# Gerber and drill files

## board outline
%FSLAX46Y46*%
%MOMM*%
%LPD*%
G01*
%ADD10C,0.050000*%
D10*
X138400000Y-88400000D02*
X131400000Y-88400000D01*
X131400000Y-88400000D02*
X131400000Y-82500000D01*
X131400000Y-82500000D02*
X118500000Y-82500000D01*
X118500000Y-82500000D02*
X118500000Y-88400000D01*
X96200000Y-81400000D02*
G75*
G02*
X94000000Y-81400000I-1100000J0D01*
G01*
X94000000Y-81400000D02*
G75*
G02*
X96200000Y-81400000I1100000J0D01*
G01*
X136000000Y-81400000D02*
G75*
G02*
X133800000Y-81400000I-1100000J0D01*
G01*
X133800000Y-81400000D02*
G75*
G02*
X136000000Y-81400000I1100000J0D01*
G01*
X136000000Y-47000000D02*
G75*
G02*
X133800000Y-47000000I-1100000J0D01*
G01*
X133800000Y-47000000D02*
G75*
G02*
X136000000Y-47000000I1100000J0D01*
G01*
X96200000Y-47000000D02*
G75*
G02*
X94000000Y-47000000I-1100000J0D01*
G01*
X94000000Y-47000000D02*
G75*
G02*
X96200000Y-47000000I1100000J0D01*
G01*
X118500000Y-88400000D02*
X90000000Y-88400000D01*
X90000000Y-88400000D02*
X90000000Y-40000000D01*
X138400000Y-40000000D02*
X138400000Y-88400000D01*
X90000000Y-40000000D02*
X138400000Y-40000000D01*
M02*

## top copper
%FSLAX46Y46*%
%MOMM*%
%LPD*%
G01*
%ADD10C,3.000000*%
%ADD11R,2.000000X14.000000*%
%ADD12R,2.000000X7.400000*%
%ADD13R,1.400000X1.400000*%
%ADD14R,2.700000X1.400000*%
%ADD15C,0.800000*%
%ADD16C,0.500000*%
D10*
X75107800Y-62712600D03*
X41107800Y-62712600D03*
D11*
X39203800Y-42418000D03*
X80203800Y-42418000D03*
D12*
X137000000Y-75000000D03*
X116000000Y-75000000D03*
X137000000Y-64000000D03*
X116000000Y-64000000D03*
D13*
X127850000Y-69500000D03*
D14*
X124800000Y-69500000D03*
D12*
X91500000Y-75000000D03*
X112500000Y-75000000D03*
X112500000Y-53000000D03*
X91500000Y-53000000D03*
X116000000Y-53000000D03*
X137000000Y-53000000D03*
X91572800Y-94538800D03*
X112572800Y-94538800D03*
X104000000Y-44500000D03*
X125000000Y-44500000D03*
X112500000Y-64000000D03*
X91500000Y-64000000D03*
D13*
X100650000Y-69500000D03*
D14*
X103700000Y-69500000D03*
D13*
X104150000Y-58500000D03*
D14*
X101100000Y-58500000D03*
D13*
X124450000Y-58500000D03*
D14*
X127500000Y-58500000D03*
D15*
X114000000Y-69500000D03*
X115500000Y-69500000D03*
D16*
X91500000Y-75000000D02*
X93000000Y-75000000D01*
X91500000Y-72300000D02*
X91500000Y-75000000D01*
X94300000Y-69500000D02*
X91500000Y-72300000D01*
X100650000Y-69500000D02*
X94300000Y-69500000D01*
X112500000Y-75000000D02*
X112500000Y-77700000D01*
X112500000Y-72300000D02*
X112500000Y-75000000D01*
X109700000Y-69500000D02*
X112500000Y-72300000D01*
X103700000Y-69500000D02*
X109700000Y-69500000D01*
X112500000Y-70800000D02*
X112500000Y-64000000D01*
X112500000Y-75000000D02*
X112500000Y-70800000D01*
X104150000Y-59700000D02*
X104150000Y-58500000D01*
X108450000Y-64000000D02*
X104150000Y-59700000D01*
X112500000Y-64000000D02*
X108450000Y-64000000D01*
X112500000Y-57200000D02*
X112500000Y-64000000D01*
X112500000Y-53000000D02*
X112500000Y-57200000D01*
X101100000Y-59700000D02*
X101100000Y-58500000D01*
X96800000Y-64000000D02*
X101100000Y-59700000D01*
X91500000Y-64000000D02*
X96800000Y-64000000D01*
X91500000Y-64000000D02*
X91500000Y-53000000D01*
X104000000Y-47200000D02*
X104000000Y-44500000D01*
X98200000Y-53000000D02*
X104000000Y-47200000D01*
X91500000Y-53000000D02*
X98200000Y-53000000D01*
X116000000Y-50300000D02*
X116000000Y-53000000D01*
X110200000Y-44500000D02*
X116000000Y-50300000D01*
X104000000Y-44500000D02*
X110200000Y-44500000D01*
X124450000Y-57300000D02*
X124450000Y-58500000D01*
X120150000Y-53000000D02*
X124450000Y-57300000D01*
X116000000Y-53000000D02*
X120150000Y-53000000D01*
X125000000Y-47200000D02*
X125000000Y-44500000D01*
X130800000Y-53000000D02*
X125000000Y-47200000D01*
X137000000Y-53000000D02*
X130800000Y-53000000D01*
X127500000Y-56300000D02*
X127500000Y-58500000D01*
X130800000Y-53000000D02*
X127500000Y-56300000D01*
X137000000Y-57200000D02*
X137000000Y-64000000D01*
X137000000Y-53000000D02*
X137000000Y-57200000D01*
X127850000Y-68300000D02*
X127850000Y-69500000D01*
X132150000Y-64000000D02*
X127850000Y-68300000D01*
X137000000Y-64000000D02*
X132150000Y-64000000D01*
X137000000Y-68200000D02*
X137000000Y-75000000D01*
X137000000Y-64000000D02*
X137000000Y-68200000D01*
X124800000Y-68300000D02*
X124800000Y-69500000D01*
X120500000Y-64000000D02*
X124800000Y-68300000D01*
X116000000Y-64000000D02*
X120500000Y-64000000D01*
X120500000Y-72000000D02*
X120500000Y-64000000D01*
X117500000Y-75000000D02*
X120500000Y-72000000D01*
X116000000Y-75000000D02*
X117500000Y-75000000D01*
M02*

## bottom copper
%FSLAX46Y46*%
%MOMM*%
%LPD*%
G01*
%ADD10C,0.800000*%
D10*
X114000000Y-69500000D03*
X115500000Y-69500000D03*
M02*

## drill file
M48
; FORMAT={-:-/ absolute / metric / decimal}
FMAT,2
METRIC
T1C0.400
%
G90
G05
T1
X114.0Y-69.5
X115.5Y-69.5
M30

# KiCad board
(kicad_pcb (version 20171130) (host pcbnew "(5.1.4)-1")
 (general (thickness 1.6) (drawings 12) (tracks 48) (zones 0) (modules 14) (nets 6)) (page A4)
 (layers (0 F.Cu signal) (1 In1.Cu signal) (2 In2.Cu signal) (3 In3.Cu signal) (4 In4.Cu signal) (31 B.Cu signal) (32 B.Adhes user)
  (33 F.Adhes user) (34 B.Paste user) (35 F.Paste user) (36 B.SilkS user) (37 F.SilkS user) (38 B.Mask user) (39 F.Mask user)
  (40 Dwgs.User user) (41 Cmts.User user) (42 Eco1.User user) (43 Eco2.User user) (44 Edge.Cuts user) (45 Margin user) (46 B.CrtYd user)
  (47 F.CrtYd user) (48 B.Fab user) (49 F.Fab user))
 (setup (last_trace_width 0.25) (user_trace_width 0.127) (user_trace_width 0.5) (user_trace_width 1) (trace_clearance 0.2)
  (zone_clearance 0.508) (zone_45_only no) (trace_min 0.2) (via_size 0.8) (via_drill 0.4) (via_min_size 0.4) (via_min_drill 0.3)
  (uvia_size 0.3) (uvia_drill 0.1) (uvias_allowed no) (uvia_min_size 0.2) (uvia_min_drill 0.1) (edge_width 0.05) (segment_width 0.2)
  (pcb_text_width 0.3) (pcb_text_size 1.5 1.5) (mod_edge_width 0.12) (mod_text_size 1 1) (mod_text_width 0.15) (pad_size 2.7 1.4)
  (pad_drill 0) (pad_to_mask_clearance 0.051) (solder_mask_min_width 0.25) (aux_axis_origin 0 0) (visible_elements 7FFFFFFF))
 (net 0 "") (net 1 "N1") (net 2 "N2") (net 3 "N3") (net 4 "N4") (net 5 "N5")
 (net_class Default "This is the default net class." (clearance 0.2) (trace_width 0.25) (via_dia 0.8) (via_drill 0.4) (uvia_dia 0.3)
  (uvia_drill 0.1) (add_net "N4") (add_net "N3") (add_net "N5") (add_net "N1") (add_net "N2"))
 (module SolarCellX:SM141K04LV (layer F.Cu) (at 35.6078 62.7126)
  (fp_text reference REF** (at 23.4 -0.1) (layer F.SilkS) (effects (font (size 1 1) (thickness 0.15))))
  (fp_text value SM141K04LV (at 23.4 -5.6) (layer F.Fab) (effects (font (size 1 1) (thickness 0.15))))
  (pad 2 smd circle (at 39.5 0) (size 3 3) (layers F.Cu F.Paste F.Mask))
  (pad 1 smd circle (at 5.5 0) (size 3 3) (layers F.Cu F.Paste F.Mask)))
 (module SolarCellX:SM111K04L (layer F.Cu) (at 81.2038 42.418 180)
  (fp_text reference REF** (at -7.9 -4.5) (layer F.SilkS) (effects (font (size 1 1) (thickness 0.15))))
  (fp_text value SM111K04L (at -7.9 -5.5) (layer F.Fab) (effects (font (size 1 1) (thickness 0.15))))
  (pad 2 smd rect (at 42 0 180) (size 2 14) (layers F.Cu F.Paste F.Mask))
  (pad 1 smd rect (at 1 0 180) (size 2 14) (layers F.Cu F.Paste F.Mask)))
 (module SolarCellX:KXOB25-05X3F (layer F.Cu) (at 116 75)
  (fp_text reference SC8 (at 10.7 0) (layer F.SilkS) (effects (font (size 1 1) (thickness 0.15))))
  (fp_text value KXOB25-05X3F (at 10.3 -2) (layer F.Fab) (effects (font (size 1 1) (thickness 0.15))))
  (pad 2 smd rect (at 21 0) (size 2 7.4) (layers F.Cu F.Paste F.Mask) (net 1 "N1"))
  (pad 1 smd rect (at 0 0) (size 2 7.4) (layers F.Cu F.Paste F.Mask) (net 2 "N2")))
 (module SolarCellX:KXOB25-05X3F (layer F.Cu) (at 116 64)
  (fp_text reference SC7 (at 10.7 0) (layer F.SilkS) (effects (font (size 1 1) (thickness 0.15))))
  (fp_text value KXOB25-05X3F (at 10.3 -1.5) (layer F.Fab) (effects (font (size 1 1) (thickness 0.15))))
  (pad 2 smd rect (at 21 0) (size 2 7.4) (layers F.Cu F.Paste F.Mask) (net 1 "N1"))
  (pad 1 smd rect (at 0 0) (size 2 7.4) (layers F.Cu F.Paste F.Mask) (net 2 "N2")))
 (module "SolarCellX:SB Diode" (layer F.Cu) (at 126 69.5)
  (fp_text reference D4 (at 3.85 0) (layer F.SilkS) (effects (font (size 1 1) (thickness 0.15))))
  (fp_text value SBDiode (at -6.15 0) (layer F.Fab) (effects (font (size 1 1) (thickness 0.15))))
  (pad 2 smd rect (at 1.85 0) (size 1.4 1.4) (layers F.Cu F.Paste F.Mask) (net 1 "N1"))
  (pad 1 smd rect (at -1.2 0) (size 2.7 1.4) (layers F.Cu F.Paste F.Mask) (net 2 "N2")))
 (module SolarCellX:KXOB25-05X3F (layer F.Cu) (at 112.5 75 180)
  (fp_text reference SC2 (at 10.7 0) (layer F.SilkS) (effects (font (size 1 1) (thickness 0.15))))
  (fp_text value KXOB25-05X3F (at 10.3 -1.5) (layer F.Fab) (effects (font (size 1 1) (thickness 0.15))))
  (pad 2 smd rect (at 21 0 180) (size 2 7.4) (layers F.Cu F.Paste F.Mask) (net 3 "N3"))
  (pad 1 smd rect (at 0 0 180) (size 2 7.4) (layers F.Cu F.Paste F.Mask) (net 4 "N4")))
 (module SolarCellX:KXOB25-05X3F (layer F.Cu) (at 91.5 53)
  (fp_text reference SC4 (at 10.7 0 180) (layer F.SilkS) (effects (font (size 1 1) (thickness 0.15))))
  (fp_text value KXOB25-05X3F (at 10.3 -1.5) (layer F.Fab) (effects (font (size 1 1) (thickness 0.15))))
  (pad 2 smd rect (at 21 0) (size 2 7.4) (layers F.Cu F.Paste F.Mask) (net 4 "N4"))
  (pad 1 smd rect (at 0 0) (size 2 7.4) (layers F.Cu F.Paste F.Mask) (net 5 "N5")))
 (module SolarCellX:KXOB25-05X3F (layer F.Cu) (at 137 53 180)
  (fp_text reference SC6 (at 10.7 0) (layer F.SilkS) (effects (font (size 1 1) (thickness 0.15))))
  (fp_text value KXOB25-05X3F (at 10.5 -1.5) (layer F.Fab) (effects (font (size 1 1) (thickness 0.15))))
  (pad 2 smd rect (at 21 0 180) (size 2 7.4) (layers F.Cu F.Paste F.Mask) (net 5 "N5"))
  (pad 1 smd rect (at 0 0 180) (size 2 7.4) (layers F.Cu F.Paste F.Mask) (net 1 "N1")))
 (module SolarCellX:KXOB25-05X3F (layer F.Cu) (at 112.5728 94.5388 180)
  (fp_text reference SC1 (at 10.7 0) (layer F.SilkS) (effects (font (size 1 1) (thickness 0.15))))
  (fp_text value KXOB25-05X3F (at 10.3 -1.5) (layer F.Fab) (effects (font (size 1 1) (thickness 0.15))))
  (pad 2 smd rect (at 21 0 180) (size 2 7.4) (layers F.Cu F.Paste F.Mask) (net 3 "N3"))
  (pad 1 smd rect (at 0 0 180) (size 2 7.4) (layers F.Cu F.Paste F.Mask) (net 4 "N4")))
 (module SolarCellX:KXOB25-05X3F (layer F.Cu) (at 125 44.5 180)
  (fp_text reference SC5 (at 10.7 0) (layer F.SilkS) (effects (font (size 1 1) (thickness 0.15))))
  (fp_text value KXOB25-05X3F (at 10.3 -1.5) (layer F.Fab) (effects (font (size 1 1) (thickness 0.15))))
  (pad 2 smd rect (at 21 0 180) (size 2 7.4) (layers F.Cu F.Paste F.Mask) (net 5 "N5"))
  (pad 1 smd rect (at 0 0 180) (size 2 7.4) (layers F.Cu F.Paste F.Mask) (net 1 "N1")))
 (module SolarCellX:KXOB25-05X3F (layer F.Cu) (at 91.5 64)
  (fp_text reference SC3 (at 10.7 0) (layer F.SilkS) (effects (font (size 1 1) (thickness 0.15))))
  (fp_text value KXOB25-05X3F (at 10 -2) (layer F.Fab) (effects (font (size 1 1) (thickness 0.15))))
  (pad 2 smd rect (at 21 0) (size 2 7.4) (layers F.Cu F.Paste F.Mask) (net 4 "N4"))
  (pad 1 smd rect (at 0 0) (size 2 7.4) (layers F.Cu F.Paste F.Mask) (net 5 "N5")))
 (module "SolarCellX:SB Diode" (layer F.Cu) (at 102.5 69.5 180)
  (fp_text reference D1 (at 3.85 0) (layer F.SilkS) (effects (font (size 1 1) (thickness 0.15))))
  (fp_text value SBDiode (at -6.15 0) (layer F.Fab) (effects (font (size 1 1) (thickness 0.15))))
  (pad 2 smd rect (at 1.85 0 180) (size 1.4 1.4) (layers F.Cu F.Paste F.Mask) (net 3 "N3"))
  (pad 1 smd rect (at -1.2 0 180) (size 2.7 1.4) (layers F.Cu F.Paste F.Mask) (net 4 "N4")))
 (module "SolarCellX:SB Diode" (layer F.Cu) (at 102.3 58.5)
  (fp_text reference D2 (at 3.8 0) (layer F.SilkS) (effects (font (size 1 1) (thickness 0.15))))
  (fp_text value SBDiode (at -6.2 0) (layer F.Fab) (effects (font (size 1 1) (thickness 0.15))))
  (pad 2 smd rect (at 1.85 0) (size 1.4 1.4) (layers F.Cu F.Paste F.Mask) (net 4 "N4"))
  (pad 1 smd rect (at -1.2 0) (size 2.7 1.4) (layers F.Cu F.Paste F.Mask) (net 5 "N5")))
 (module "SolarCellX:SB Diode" (layer F.Cu) (at 126.3 58.5 180)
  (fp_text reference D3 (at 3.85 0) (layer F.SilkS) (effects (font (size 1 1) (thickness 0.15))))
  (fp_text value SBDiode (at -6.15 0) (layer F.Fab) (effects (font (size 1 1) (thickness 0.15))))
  (pad 2 smd rect (at 1.85 0 180) (size 1.4 1.4) (layers F.Cu F.Paste F.Mask) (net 5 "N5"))
  (pad 1 smd rect (at -1.2 0 180) (size 2.7 1.4) (layers F.Cu F.Paste F.Mask) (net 1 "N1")))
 (gr_line (start 138.4 88.4) (end 131.4 88.4) (layer Edge.Cuts) (width 0.05))
 (gr_line (start 131.4 88.4) (end 131.4 82.5) (layer Edge.Cuts) (width 0.05))
 (gr_line (start 131.4 82.5) (end 118.5 82.5) (layer Edge.Cuts) (width 0.05))
 (gr_line (start 118.5 82.5) (end 118.5 88.4) (layer Edge.Cuts) (width 0.05))
 (gr_circle (center 95.1 81.4) (end 96.2 81.4) (layer Edge.Cuts) (width 0.05))
 (gr_circle (center 134.9 81.4) (end 136 81.4) (layer Edge.Cuts) (width 0.05))
 (gr_circle (center 134.9 47) (end 136 47) (layer Edge.Cuts) (width 0.05))
 (gr_circle (center 95.1 47) (end 96.2 47) (layer Edge.Cuts) (width 0.05))
 (gr_line (start 118.5 88.4) (end 90 88.4) (layer Edge.Cuts) (width 0.05))
 (gr_line (start 90 88.4) (end 90 40) (layer Edge.Cuts) (width 0.05))
 (gr_line (start 138.4 40) (end 138.4 88.4) (layer Edge.Cuts) (width 0.05))
 (gr_line (start 90 40) (end 138.4 40) (layer Edge.Cuts) (width 0.05))
 (via (at 114 69.5) (size 0.8) (drill 0.4) (layers F.Cu B.Cu) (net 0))
 (via (at 115.5 69.5) (size 0.8) (drill 0.4) (layers F.Cu B.Cu) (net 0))
 (segment (start 91.5 75) (end 93 75) (width 0.5) (layer F.Cu) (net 3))
 (segment (start 91.5 72.3) (end 91.5 75) (width 0.5) (layer F.Cu) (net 3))
 (segment (start 94.3 69.5) (end 91.5 72.3) (width 0.5) (layer F.Cu) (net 3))
 (segment (start 100.65 69.5) (end 94.3 69.5) (width 0.5) (layer F.Cu) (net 3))
 (segment (start 112.5 75) (end 112.5 77.7) (width 0.5) (layer F.Cu) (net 4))
 (segment (start 112.5 72.3) (end 112.5 75) (width 0.5) (layer F.Cu) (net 4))
 (segment (start 109.7 69.5) (end 112.5 72.3) (width 0.5) (layer F.Cu) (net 4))
 (segment (start 103.7 69.5) (end 109.7 69.5) (width 0.5) (layer F.Cu) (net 4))
 (segment (start 112.5 70.8) (end 112.5 64) (width 0.5) (layer F.Cu) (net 4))
 (segment (start 112.5 75) (end 112.5 70.8) (width 0.5) (layer F.Cu) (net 4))
 (segment (start 104.15 59.7) (end 104.15 58.5) (width 0.5) (layer F.Cu) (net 4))
 (segment (start 108.45 64) (end 104.15 59.7) (width 0.5) (layer F.Cu) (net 4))
 (segment (start 112.5 64) (end 108.45 64) (width 0.5) (layer F.Cu) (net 4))
 (segment (start 112.5 57.2) (end 112.5 64) (width 0.5) (layer F.Cu) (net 4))
 (segment (start 112.5 53) (end 112.5 57.2) (width 0.5) (layer F.Cu) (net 4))
 (segment (start 101.1 59.7) (end 101.1 58.5) (width 0.5) (layer F.Cu) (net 5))
 (segment (start 96.8 64) (end 101.1 59.7) (width 0.5) (layer F.Cu) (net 5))
 (segment (start 91.5 64) (end 96.8 64) (width 0.5) (layer F.Cu) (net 5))
 (segment (start 91.5 64) (end 91.5 53) (width 0.5) (layer F.Cu) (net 5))
 (segment (start 104 47.2) (end 104 44.5) (width 0.5) (layer F.Cu) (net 5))
 (segment (start 98.2 53) (end 104 47.2) (width 0.5) (layer F.Cu) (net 5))
 (segment (start 91.5 53) (end 98.2 53) (width 0.5) (layer F.Cu) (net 5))
 (segment (start 116 50.3) (end 116 53) (width 0.5) (layer F.Cu) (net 5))
 (segment (start 110.2 44.5) (end 116 50.3) (width 0.5) (layer F.Cu) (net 5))
 (segment (start 104 44.5) (end 110.2 44.5) (width 0.5) (layer F.Cu) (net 5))
 (segment (start 124.45 57.3) (end 124.45 58.5) (width 0.5) (layer F.Cu) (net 5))
 (segment (start 120.15 53) (end 124.45 57.3) (width 0.5) (layer F.Cu) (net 5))
 (segment (start 116 53) (end 120.15 53) (width 0.5) (layer F.Cu) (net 5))
 (segment (start 125 47.2) (end 125 44.5) (width 0.5) (layer F.Cu) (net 1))
 (segment (start 130.8 53) (end 125 47.2) (width 0.5) (layer F.Cu) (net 1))
 (segment (start 137 53) (end 130.8 53) (width 0.5) (layer F.Cu) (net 1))
 (segment (start 127.5 56.3) (end 127.5 58.5) (width 0.5) (layer F.Cu) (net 1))
 (segment (start 130.8 53) (end 127.5 56.3) (width 0.5) (layer F.Cu) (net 1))
 (segment (start 137 57.2) (end 137 64) (width 0.5) (layer F.Cu) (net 1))
 (segment (start 137 53) (end 137 57.2) (width 0.5) (layer F.Cu) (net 1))
 (segment (start 127.85 68.3) (end 127.85 69.5) (width 0.5) (layer F.Cu) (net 1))
 (segment (start 132.15 64) (end 127.85 68.3) (width 0.5) (layer F.Cu) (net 1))
 (segment (start 137 64) (end 132.15 64) (width 0.5) (layer F.Cu) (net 1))
 (segment (start 137 68.2) (end 137 75) (width 0.5) (layer F.Cu) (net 1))
 (segment (start 137 64) (end 137 68.2) (width 0.5) (layer F.Cu) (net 1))
 (segment (start 124.8 68.3) (end 124.8 69.5) (width 0.5) (layer F.Cu) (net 2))
 (segment (start 120.5 64) (end 124.8 68.3) (width 0.5) (layer F.Cu) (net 2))
 (segment (start 116 64) (end 120.5 64) (width 0.5) (layer F.Cu) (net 2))
 (segment (start 120.5 72) (end 120.5 64) (width 0.5) (layer F.Cu) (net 2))
 (segment (start 117.5 75) (end 120.5 72) (width 0.5) (layer F.Cu) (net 2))
 (segment (start 116 75) (end 117.5 75) (width 0.5) (layer F.Cu) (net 2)))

